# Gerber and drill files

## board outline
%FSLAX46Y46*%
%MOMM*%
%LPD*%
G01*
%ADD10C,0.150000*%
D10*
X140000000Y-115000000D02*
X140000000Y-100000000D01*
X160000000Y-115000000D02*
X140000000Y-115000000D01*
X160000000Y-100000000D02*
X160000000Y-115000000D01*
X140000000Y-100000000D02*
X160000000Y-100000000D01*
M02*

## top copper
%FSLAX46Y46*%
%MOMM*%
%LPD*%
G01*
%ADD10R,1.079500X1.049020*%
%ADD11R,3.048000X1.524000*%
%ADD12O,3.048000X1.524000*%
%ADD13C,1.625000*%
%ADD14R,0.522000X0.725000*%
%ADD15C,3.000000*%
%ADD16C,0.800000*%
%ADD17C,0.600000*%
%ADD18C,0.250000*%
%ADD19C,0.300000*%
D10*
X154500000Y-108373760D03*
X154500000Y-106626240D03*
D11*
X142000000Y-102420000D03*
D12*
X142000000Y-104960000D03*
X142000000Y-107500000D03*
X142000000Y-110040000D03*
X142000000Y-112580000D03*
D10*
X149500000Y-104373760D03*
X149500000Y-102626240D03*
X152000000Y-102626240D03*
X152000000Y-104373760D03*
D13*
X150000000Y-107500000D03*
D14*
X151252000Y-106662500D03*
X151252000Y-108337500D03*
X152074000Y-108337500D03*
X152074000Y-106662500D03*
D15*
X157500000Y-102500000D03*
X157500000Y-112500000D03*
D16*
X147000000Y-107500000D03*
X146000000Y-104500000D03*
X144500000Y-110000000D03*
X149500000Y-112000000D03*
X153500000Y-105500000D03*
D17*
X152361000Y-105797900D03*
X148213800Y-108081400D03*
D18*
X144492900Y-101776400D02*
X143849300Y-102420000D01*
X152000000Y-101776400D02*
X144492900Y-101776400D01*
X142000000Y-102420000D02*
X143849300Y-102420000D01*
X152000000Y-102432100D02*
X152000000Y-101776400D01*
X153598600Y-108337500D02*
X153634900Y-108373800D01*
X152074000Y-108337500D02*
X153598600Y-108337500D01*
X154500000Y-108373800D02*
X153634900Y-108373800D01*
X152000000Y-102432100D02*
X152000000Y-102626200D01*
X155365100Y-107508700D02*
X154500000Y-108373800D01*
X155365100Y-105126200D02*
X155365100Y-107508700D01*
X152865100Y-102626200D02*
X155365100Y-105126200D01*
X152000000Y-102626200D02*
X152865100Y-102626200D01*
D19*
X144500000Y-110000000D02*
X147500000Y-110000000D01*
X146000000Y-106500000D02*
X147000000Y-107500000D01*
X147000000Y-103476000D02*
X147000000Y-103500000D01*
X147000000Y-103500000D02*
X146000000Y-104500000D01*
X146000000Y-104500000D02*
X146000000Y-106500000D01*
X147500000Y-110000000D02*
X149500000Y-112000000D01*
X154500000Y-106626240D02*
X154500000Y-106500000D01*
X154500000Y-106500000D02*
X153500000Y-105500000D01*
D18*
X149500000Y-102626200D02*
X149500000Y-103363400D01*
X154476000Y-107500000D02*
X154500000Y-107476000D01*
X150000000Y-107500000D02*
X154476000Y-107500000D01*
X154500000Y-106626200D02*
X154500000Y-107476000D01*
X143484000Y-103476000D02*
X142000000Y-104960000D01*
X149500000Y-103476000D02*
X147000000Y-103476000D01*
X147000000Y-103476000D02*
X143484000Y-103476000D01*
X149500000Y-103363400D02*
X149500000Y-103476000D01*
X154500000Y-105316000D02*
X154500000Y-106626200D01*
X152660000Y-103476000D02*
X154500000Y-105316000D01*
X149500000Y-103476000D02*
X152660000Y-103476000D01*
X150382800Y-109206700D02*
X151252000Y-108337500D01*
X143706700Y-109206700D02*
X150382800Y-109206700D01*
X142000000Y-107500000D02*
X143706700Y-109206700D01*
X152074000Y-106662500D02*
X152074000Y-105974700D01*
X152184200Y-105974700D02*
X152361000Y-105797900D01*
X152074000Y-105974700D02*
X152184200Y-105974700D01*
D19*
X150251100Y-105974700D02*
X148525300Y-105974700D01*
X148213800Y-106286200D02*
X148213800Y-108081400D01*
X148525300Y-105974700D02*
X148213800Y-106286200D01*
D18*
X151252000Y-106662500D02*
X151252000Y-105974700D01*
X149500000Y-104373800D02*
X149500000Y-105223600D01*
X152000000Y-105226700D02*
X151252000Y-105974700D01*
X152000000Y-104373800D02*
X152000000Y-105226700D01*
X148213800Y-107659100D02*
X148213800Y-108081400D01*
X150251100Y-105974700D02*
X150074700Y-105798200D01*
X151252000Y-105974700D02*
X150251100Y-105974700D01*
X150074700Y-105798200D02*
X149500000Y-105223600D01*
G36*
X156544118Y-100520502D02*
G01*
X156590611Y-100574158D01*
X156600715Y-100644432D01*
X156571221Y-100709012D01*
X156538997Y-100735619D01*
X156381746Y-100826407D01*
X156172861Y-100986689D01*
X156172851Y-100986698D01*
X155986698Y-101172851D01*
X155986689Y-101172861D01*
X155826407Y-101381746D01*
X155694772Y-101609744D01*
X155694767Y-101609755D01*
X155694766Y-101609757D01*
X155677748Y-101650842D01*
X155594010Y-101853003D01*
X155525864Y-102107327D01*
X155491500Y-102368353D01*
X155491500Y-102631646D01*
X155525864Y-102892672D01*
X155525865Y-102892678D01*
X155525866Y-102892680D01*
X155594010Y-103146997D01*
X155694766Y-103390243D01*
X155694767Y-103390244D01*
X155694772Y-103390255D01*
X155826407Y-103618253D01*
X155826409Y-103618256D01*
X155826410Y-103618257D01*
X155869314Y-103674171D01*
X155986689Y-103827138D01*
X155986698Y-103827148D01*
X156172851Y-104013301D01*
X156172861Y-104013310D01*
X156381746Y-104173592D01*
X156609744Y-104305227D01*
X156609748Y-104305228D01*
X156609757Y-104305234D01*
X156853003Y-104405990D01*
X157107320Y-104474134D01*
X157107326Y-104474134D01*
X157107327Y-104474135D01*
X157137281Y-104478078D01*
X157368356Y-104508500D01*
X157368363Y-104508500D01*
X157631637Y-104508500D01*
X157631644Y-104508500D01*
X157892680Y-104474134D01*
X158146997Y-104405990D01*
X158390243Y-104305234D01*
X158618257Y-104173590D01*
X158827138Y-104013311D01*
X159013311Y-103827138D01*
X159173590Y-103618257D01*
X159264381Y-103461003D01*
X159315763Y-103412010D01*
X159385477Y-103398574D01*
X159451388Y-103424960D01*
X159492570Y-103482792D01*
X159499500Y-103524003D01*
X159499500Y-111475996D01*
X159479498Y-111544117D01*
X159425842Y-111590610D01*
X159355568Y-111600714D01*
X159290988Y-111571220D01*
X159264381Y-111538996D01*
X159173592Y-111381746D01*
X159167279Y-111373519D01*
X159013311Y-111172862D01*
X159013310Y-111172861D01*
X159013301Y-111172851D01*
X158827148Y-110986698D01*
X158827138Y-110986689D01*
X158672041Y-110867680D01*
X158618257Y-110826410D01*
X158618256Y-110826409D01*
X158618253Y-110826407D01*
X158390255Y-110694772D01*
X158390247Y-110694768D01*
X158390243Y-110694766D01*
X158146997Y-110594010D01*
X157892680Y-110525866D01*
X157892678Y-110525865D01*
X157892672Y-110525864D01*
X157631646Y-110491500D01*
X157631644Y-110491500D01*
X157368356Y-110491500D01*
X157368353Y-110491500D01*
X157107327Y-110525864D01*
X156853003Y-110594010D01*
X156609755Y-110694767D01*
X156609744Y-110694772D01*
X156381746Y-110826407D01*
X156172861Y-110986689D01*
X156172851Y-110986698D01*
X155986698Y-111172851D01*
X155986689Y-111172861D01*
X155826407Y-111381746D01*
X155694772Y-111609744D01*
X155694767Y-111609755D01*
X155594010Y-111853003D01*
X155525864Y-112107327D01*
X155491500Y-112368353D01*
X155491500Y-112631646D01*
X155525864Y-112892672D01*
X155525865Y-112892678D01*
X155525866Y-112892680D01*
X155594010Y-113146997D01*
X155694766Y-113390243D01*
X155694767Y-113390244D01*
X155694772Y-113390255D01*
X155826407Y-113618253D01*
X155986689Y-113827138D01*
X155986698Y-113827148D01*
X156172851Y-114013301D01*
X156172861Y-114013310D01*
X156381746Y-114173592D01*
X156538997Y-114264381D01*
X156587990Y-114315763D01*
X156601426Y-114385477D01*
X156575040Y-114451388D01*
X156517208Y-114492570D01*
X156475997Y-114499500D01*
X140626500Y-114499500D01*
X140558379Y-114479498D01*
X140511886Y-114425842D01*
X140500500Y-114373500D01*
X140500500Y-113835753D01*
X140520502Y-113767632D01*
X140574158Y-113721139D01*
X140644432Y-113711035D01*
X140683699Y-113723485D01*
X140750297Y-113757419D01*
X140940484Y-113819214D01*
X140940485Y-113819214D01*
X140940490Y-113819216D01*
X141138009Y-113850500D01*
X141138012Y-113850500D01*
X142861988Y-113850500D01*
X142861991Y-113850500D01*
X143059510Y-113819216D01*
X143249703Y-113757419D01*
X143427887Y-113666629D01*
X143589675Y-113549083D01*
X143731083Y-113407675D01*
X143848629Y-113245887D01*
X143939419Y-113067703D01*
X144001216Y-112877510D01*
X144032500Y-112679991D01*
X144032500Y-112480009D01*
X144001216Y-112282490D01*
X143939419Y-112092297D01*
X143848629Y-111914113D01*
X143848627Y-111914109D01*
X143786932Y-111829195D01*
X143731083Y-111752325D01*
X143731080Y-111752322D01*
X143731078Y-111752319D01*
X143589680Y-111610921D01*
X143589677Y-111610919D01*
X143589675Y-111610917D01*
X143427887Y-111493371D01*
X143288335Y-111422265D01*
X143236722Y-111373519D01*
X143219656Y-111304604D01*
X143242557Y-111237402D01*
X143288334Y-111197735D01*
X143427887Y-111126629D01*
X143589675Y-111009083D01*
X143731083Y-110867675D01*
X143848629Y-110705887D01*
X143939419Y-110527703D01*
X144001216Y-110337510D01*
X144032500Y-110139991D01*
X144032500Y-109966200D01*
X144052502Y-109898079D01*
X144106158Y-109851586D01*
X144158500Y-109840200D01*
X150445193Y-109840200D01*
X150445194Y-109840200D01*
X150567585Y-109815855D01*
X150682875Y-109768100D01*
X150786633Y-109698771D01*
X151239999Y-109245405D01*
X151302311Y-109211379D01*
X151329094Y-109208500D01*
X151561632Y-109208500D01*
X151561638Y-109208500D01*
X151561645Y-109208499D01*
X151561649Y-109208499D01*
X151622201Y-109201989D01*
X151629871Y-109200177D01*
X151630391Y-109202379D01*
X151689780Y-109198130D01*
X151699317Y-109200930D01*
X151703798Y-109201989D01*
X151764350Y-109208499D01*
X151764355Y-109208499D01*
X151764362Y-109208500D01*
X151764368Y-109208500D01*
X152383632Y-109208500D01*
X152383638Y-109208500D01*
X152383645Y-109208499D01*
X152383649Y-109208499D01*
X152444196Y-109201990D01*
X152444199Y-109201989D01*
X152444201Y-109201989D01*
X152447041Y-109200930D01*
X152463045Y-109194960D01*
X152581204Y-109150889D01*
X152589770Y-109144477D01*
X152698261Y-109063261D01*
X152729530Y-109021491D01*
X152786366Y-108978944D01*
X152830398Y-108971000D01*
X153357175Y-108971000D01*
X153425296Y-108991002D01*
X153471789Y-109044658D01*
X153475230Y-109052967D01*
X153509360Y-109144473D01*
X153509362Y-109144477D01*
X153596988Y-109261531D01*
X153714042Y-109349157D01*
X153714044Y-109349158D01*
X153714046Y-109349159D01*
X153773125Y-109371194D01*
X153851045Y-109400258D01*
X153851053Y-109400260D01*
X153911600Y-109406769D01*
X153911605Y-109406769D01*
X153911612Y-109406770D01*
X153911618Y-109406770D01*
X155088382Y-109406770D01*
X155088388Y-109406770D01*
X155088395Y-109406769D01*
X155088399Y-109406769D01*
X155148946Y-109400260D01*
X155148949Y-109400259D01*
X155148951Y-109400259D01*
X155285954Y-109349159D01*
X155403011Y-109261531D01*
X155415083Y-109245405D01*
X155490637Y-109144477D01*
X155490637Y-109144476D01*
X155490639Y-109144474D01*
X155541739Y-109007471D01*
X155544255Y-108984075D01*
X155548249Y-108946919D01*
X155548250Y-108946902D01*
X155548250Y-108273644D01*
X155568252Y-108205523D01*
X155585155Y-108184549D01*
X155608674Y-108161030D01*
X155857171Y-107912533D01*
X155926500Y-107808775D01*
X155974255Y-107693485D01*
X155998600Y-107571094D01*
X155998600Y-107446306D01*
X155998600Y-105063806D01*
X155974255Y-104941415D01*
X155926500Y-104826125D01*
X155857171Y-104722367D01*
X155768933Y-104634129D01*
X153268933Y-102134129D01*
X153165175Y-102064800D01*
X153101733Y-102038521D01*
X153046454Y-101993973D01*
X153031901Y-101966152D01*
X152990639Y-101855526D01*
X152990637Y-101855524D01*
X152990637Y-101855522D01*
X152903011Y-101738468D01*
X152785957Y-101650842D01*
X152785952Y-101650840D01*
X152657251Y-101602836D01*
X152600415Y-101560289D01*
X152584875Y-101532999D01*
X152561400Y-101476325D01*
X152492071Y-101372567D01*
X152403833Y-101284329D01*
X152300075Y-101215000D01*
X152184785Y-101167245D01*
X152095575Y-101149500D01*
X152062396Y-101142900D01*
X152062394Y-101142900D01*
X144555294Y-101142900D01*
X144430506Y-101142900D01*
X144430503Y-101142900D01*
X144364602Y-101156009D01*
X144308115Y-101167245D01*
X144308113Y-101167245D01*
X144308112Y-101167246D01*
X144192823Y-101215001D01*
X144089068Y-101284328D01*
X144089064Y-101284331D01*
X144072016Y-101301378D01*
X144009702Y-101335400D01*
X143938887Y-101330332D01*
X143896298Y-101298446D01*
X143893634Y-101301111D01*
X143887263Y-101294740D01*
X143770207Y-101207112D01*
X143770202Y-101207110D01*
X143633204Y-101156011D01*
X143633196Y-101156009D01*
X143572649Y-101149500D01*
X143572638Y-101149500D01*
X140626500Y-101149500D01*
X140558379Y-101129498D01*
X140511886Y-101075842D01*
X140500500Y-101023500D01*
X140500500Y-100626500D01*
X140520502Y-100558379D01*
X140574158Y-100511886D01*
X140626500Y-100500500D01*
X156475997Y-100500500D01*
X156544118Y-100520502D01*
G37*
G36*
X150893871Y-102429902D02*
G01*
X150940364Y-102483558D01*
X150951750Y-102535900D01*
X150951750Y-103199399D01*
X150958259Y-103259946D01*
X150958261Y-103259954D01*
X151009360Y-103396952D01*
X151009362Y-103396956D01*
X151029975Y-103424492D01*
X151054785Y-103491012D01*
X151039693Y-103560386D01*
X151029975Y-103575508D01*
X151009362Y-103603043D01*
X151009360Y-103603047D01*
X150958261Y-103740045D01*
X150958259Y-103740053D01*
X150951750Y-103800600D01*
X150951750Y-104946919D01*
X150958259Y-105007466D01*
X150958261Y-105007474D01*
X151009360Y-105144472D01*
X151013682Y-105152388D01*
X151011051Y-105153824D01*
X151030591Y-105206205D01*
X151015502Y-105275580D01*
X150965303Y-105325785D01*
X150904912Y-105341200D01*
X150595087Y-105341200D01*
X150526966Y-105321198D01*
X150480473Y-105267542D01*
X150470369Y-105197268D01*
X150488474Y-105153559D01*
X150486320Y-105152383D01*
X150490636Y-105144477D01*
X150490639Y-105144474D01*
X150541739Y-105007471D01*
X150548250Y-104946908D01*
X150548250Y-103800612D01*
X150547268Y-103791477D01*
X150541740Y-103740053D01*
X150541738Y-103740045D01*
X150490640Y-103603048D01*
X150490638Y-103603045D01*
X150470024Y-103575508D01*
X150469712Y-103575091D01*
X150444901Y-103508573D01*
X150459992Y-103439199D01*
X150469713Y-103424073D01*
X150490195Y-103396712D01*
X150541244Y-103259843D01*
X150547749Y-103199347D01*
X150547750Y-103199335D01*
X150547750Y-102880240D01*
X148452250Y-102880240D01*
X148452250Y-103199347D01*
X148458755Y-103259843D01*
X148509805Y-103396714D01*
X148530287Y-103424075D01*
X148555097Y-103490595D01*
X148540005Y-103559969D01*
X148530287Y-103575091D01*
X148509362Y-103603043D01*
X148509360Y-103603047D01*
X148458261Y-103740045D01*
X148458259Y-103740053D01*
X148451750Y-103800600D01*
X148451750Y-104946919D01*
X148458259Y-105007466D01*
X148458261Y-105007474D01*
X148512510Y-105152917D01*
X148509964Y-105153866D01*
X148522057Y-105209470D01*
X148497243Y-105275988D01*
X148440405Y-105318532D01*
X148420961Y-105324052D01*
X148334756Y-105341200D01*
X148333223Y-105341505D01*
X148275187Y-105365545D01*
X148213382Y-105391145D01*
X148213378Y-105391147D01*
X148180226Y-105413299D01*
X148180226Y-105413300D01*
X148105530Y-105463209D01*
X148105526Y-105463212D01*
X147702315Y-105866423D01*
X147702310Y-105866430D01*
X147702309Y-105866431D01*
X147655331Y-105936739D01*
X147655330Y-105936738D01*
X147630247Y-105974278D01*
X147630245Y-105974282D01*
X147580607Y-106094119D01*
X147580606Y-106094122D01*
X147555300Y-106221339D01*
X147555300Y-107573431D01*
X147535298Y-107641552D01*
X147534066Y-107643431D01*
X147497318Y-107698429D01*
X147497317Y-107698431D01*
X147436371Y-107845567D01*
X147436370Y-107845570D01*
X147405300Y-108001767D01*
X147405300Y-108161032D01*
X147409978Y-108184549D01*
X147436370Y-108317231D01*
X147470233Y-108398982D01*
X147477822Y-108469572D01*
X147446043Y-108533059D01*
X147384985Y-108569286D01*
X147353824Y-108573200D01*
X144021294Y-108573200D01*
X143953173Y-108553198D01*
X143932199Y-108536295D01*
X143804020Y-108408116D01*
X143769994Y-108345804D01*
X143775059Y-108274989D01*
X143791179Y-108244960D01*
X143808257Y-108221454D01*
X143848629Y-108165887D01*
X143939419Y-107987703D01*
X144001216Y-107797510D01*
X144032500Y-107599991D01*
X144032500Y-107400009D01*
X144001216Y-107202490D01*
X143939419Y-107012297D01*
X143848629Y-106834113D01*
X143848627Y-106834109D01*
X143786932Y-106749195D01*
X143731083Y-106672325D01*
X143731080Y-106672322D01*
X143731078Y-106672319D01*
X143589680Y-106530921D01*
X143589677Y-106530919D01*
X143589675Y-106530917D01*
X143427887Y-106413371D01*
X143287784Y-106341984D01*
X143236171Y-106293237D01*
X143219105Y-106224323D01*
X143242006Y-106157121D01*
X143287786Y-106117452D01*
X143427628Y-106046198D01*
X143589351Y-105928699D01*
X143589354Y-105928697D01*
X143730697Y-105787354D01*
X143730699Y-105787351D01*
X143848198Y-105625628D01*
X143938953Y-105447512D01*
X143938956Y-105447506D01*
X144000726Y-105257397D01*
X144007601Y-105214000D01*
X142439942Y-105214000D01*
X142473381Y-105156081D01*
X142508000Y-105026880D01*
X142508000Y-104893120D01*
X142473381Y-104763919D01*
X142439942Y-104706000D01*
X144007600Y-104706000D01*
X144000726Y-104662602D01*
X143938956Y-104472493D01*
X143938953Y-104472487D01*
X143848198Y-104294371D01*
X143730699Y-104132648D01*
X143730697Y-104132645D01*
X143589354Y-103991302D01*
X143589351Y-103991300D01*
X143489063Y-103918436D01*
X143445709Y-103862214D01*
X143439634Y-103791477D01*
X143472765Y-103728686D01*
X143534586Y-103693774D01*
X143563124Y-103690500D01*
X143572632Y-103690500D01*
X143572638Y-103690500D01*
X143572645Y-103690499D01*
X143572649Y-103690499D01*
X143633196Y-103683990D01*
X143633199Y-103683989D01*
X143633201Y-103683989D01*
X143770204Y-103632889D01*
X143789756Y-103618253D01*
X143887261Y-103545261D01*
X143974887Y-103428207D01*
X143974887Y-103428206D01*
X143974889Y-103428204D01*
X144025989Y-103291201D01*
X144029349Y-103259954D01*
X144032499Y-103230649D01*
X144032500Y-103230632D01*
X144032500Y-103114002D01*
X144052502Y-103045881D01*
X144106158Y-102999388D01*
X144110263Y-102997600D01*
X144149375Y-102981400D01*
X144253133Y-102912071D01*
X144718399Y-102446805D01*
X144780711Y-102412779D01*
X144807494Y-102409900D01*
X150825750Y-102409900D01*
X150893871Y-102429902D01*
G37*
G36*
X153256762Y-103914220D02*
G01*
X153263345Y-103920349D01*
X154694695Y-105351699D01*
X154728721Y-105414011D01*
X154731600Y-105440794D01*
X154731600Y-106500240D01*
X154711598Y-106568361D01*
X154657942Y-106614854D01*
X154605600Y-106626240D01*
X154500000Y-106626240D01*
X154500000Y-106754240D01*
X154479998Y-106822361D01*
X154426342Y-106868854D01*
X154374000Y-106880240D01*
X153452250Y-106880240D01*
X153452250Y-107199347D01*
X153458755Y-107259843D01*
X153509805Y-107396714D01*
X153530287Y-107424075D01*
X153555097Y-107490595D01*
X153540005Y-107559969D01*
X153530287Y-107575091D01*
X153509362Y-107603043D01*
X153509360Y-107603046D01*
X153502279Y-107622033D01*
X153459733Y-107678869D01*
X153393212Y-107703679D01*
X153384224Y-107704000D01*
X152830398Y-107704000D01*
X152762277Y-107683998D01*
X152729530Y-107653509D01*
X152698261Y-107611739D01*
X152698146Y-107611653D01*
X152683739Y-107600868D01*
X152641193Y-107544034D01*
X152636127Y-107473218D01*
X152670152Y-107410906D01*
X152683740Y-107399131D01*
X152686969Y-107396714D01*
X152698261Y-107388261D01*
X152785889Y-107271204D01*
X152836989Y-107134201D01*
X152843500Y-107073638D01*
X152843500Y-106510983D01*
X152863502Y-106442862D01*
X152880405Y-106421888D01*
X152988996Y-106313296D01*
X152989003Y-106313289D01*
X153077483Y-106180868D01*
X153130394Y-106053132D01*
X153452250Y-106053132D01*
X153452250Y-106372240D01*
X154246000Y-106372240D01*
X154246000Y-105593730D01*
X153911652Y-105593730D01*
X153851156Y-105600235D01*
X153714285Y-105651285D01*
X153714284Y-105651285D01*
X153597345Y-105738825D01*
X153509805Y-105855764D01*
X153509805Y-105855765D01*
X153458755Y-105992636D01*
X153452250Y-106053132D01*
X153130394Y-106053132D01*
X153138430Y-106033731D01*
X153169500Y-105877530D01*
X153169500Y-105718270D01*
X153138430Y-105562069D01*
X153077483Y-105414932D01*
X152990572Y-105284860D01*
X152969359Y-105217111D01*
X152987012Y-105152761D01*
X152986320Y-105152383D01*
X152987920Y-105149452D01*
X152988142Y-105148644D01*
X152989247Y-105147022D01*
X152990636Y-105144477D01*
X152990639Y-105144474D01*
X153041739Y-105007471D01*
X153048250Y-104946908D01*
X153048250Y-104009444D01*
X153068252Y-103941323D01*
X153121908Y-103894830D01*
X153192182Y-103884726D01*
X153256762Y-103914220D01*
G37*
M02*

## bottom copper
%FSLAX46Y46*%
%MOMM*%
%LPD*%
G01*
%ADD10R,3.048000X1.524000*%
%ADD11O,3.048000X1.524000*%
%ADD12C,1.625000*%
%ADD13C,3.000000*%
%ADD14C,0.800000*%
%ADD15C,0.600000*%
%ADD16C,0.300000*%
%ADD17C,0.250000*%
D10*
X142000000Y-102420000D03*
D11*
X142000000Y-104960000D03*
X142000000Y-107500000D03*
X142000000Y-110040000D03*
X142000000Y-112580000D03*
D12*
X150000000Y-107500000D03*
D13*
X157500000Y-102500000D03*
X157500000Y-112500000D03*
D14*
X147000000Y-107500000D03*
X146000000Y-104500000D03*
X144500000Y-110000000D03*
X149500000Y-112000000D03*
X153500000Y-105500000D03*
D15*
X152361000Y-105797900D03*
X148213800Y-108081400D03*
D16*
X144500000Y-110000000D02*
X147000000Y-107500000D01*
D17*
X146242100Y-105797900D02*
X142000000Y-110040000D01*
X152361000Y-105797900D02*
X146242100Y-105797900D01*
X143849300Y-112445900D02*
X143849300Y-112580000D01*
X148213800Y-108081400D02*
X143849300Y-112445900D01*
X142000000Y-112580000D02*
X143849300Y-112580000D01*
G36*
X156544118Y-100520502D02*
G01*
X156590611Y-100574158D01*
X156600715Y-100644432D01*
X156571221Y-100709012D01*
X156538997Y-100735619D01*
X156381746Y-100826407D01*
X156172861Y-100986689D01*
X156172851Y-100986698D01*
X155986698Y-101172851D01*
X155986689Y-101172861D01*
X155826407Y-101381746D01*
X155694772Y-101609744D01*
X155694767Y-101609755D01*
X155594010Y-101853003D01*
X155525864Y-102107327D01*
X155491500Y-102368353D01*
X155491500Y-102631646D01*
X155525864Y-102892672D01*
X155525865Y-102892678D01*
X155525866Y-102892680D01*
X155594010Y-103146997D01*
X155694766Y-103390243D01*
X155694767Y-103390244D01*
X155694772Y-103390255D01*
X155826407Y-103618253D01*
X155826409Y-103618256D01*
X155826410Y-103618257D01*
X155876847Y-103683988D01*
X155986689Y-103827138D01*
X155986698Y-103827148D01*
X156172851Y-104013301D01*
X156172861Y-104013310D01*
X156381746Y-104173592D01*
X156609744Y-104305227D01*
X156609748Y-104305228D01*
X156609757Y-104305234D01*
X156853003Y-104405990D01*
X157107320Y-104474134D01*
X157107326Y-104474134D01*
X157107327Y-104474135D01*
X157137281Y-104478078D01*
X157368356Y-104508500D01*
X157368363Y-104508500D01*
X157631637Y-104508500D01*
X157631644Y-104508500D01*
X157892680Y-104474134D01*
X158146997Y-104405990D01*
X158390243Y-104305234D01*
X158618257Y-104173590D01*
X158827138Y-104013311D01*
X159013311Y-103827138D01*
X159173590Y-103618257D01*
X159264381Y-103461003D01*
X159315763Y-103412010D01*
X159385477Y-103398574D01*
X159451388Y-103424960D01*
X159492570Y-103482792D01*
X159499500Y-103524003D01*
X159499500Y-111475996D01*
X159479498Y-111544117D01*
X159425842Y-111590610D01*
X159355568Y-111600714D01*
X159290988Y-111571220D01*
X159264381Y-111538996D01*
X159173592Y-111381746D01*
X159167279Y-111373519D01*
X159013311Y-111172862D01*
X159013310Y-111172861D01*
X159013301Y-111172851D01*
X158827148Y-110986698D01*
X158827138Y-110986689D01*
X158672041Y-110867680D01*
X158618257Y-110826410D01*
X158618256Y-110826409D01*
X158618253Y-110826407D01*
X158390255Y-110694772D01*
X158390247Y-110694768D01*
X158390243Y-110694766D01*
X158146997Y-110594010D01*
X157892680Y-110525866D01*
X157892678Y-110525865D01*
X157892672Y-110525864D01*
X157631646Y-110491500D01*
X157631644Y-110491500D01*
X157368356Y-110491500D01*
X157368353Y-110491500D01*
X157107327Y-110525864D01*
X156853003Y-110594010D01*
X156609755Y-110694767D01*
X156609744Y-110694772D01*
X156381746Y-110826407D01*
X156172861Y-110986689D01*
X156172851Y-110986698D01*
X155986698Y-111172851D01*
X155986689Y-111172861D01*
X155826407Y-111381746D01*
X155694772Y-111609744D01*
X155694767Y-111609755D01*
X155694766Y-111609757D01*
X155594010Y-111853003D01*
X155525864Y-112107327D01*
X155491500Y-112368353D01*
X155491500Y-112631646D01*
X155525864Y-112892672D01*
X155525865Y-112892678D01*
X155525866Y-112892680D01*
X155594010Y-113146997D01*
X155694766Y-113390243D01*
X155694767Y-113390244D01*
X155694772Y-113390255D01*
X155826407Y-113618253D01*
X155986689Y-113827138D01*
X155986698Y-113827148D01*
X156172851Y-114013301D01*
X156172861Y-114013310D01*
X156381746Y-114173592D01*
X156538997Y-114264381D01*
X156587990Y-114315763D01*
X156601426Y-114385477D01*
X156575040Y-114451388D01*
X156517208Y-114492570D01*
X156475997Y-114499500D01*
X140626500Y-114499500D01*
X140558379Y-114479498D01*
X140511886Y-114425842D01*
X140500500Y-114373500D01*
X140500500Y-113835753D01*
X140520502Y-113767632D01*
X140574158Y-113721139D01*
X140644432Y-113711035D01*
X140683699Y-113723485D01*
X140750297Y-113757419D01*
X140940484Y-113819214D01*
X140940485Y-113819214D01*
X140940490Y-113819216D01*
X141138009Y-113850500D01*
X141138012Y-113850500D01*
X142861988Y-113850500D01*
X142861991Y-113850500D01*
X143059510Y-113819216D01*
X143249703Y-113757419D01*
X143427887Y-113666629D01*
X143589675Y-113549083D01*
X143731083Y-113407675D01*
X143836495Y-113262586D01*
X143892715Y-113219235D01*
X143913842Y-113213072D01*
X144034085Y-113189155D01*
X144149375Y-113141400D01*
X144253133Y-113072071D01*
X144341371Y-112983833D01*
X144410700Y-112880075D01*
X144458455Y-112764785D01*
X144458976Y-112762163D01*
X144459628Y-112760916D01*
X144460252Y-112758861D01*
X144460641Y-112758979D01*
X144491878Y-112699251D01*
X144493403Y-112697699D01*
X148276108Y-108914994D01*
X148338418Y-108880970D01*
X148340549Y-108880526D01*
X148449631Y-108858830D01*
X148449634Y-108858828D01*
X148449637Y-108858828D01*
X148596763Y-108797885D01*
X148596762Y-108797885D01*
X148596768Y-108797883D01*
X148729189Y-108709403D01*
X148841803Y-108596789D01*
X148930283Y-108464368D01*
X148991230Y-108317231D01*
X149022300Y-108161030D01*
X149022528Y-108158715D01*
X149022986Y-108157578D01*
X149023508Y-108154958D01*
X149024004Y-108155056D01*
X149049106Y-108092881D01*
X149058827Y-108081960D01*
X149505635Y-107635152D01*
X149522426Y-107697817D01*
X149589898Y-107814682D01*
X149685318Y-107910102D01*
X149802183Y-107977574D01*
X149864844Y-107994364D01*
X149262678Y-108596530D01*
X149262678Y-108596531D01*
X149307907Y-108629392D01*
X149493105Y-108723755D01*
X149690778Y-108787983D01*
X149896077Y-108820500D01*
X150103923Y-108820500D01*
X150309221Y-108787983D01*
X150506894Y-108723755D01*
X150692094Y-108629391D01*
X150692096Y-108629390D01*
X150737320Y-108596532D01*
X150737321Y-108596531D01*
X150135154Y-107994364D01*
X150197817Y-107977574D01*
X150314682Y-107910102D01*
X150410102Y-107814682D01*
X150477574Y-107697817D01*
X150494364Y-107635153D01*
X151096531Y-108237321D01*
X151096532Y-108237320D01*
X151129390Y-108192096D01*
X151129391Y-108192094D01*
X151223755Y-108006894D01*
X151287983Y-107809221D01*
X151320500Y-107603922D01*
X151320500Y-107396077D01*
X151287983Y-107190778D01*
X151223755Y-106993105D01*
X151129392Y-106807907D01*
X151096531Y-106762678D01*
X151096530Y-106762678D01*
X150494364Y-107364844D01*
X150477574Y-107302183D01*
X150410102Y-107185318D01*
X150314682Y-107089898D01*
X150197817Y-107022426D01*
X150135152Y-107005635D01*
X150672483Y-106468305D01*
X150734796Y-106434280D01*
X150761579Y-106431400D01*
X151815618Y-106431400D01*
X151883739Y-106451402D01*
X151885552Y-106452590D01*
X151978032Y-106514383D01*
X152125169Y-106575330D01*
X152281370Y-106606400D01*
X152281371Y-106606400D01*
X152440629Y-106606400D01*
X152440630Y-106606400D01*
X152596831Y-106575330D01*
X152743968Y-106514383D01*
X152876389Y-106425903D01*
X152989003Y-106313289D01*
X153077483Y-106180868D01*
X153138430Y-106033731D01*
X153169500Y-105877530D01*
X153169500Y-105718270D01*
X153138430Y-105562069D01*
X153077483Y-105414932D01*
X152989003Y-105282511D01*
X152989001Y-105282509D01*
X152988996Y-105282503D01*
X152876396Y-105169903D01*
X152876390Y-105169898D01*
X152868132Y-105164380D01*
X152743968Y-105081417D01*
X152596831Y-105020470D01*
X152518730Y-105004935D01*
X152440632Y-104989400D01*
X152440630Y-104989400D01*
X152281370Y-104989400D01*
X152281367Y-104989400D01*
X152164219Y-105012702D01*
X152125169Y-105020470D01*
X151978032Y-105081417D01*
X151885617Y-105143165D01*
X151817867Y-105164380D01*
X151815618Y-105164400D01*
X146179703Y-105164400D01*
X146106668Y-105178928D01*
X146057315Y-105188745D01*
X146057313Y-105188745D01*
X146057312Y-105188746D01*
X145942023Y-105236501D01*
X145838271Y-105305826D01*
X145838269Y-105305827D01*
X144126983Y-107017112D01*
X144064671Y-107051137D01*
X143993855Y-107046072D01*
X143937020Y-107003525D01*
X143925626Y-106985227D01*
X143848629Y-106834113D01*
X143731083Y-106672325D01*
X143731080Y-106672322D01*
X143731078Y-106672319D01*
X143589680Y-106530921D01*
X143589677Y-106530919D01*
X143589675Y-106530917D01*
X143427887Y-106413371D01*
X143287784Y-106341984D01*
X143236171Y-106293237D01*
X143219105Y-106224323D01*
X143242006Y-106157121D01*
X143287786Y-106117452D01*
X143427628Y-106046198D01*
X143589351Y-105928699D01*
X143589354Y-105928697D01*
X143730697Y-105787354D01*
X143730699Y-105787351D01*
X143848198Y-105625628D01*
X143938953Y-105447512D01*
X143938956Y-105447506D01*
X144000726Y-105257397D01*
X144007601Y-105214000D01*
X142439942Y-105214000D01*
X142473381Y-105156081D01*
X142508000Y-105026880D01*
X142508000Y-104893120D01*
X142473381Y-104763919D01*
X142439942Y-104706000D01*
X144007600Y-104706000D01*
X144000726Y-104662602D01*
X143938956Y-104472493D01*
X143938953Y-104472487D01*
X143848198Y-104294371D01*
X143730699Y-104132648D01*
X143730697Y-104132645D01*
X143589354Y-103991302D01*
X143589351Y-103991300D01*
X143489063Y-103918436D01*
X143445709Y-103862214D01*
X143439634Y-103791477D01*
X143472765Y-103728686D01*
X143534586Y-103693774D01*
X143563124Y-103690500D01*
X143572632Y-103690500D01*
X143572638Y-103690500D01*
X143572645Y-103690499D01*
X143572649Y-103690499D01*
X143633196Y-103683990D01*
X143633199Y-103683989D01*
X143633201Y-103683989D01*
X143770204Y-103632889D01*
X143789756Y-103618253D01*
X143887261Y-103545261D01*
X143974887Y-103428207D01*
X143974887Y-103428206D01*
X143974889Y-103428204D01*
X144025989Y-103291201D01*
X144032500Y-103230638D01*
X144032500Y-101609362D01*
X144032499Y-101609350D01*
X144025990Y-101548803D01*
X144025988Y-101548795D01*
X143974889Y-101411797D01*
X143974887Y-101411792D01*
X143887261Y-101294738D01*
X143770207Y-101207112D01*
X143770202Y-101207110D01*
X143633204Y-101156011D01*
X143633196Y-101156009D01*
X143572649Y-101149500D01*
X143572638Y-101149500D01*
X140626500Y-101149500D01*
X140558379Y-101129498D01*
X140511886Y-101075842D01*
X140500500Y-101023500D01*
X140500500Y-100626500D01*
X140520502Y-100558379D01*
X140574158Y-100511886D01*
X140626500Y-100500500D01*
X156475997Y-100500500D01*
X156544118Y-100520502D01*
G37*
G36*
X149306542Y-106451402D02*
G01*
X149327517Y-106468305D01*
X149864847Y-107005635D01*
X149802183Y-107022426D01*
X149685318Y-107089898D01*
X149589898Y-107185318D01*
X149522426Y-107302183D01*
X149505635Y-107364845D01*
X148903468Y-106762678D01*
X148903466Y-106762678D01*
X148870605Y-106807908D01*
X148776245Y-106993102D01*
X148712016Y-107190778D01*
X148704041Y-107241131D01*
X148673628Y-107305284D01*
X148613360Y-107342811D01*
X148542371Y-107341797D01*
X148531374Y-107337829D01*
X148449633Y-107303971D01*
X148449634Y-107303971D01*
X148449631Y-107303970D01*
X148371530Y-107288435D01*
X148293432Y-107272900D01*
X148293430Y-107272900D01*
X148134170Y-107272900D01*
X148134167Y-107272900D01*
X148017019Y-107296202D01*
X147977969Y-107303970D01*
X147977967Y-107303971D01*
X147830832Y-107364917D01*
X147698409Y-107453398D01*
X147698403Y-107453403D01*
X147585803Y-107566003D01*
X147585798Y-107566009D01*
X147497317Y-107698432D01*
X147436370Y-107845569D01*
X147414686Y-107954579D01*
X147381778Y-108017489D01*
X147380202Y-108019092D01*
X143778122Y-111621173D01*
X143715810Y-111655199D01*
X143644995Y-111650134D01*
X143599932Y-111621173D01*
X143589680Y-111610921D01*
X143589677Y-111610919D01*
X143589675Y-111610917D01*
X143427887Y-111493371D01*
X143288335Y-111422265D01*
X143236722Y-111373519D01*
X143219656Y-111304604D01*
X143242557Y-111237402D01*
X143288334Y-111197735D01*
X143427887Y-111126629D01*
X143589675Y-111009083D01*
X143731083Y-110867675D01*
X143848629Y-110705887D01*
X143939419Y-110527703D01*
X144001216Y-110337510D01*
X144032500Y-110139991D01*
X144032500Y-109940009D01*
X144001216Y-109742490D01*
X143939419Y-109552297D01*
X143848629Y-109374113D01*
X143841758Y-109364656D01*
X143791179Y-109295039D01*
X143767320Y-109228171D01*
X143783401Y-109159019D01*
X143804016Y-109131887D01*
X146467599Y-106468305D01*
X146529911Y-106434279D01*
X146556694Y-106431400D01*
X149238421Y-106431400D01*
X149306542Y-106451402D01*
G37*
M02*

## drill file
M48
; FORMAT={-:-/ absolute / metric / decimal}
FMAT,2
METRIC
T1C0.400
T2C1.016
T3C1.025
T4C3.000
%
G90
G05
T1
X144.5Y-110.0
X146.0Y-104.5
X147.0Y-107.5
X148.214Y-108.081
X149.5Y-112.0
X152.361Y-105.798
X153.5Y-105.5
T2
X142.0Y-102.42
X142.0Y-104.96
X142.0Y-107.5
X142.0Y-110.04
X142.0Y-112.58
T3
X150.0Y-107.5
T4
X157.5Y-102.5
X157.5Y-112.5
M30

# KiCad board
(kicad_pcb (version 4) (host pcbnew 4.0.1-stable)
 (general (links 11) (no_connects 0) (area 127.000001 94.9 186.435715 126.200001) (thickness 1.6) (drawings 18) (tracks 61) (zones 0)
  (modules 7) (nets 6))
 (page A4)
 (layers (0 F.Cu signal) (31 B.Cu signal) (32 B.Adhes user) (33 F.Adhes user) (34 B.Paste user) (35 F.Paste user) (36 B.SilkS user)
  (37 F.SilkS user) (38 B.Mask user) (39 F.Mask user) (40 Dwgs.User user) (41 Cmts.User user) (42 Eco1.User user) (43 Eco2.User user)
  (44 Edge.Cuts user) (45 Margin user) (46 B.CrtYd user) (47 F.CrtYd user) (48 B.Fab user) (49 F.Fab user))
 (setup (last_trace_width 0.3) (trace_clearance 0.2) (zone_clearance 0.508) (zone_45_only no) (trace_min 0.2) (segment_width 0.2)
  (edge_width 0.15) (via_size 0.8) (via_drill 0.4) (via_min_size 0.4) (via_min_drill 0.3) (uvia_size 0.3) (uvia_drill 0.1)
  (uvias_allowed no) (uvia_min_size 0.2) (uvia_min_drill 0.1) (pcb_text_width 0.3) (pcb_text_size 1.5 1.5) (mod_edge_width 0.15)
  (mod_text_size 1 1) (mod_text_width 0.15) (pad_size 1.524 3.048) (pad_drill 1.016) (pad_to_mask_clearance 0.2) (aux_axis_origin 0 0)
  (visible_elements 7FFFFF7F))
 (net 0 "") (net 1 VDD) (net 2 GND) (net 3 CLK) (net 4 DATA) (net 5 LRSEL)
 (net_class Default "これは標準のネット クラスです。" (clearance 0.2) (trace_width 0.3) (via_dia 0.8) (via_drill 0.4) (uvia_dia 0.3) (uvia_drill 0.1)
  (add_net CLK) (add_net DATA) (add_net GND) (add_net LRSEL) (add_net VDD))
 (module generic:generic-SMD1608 (layer F.Cu) (at 154.5 107.5 90)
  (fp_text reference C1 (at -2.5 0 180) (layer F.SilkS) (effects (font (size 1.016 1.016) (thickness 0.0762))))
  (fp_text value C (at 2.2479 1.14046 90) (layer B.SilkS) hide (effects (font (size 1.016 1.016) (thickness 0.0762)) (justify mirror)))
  (pad 1 smd rect (at -0.87376 0 90) (size 1.04902 1.0795) (layers F.Cu F.Paste F.Mask) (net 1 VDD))
  (pad 2 smd rect (at 0.87376 0 90) (size 1.04902 1.0795) (layers F.Cu F.Paste F.Mask) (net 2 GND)))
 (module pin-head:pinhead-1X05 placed (layer F.Cu) (at 142 107.5 270)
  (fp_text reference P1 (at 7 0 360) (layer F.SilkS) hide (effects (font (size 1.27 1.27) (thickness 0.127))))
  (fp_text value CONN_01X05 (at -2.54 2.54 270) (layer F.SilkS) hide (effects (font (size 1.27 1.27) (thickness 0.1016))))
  (pad 1 thru_hole rect (at -5.08 0 90) (size 1.524 3.048) (drill 1.016) (layers *.Cu *.Paste *.Mask F.SilkS) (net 1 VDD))
  (pad 2 thru_hole oval (at -2.54 0 90) (size 1.524 3.048) (drill 1.016) (layers *.Cu *.Paste *.Mask F.SilkS) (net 2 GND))
  (pad 3 thru_hole oval (at 0 0 90) (size 1.524 3.048) (drill 1.016) (layers *.Cu *.Paste *.Mask F.SilkS) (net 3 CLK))
  (pad 4 thru_hole oval (at 2.54 0 90) (size 1.524 3.048) (drill 1.016) (layers *.Cu *.Paste *.Mask F.SilkS) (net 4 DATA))
  (pad 5 thru_hole oval (at 5.08 0 90) (size 1.524 3.048) (drill 1.016) (layers *.Cu *.Paste *.Mask F.SilkS) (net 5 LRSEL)))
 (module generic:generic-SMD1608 (layer F.Cu) (at 149.5 103.5 90)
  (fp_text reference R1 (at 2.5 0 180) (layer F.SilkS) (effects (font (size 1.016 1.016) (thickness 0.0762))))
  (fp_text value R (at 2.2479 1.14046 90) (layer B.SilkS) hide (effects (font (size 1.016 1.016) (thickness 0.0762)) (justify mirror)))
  (pad 1 smd rect (at -0.87376 0 90) (size 1.04902 1.0795) (layers F.Cu F.Paste F.Mask) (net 5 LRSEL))
  (pad 2 smd rect (at 0.87376 0 90) (size 1.04902 1.0795) (layers F.Cu F.Paste F.Mask) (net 2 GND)))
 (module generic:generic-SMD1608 (layer F.Cu) (at 152 103.5 270)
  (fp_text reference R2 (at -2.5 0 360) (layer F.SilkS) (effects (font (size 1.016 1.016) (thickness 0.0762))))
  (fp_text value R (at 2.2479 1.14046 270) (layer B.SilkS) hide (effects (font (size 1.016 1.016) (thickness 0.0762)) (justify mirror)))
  (pad 1 smd rect (at -0.87376 0 270) (size 1.04902 1.0795) (layers F.Cu F.Paste F.Mask) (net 1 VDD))
  (pad 2 smd rect (at 0.87376 0 270) (size 1.04902 1.0795) (layers F.Cu F.Paste F.Mask) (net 5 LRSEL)))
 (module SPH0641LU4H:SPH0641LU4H (layer F.Cu) (at 150 107.5 270)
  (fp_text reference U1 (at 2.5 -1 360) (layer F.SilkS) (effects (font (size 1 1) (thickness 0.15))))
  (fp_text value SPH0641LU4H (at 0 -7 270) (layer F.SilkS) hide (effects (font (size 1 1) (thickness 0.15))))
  (pad 3 thru_hole circle (at 0 0 270) (size 1.625 1.625) (drill 1.025) (layers *.Cu *.Mask F.SilkS) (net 2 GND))
  (pad 2 smd rect (at -0.8375 -1.252 270) (size 0.725 0.522) (layers F.Cu F.Paste F.Mask) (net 5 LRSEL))
  (pad 4 smd rect (at 0.8375 -1.252 270) (size 0.725 0.522) (layers F.Cu F.Paste F.Mask) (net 3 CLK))
  (pad 5 smd rect (at 0.8375 -2.074 270) (size 0.725 0.522) (layers F.Cu F.Paste F.Mask) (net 1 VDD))
  (pad 1 smd rect (at -0.8375 -2.074 270) (size 0.725 0.522) (layers F.Cu F.Paste F.Mask) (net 4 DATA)))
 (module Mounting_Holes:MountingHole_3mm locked (layer F.Cu) (at 157.5 102.5)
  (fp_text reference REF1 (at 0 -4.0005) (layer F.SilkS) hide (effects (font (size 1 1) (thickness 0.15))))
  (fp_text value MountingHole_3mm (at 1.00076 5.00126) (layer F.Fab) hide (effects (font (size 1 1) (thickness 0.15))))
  (pad 1 thru_hole circle (at 0 0) (size 3 3) (drill 3) (layers)))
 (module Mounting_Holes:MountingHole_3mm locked (layer F.Cu) (at 157.5 112.5)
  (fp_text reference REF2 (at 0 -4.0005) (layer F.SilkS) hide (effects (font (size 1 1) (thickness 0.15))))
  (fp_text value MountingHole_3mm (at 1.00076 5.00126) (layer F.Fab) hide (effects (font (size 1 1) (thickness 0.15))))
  (pad 1 thru_hole circle (at 0 0) (size 3 3) (drill 3) (layers)))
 (gr_line (start 140 115) (end 140 100) (angle 90) (layer Edge.Cuts) (width 0.15))
 (gr_line (start 160 115) (end 140 115) (angle 90) (layer Edge.Cuts) (width 0.15))
 (gr_line (start 160 100) (end 160 115) (angle 90) (layer Edge.Cuts) (width 0.15))
 (gr_line (start 140 100) (end 160 100) (angle 90) (layer Edge.Cuts) (width 0.15))
 (segment (start 144.4929 101.7764) (end 143.8493 102.42) (width 0.25) (layer F.Cu) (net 1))
 (segment (start 152 101.7764) (end 144.4929 101.7764) (width 0.25) (layer F.Cu) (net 1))
 (segment (start 142 102.42) (end 143.8493 102.42) (width 0.25) (layer F.Cu) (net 1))
 (segment (start 152 102.4321) (end 152 101.7764) (width 0.25) (layer F.Cu) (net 1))
 (segment (start 153.5986 108.3375) (end 153.6349 108.3738) (width 0.25) (layer F.Cu) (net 1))
 (segment (start 152.074 108.3375) (end 153.5986 108.3375) (width 0.25) (layer F.Cu) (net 1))
 (segment (start 154.5 108.3738) (end 153.6349 108.3738) (width 0.25) (layer F.Cu) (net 1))
 (segment (start 152 102.4321) (end 152 102.6262) (width 0.25) (layer F.Cu) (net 1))
 (segment (start 155.3651 107.5087) (end 154.5 108.3738) (width 0.25) (layer F.Cu) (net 1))
 (segment (start 155.3651 105.1262) (end 155.3651 107.5087) (width 0.25) (layer F.Cu) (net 1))
 (segment (start 152.8651 102.6262) (end 155.3651 105.1262) (width 0.25) (layer F.Cu) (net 1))
 (segment (start 152 102.6262) (end 152.8651 102.6262) (width 0.25) (layer F.Cu) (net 1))
 (segment (start 144.5 110) (end 147.5 110) (width 0.3) (layer F.Cu) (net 2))
 (segment (start 144.5 110) (end 147 107.5) (width 0.3) (layer B.Cu) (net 2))
 (segment (start 146 106.5) (end 147 107.5) (width 0.3) (layer F.Cu) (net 2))
 (via (at 147 107.5) (size 0.8) (drill 0.4) (layers F.Cu B.Cu) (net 2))
 (segment (start 147 103.476) (end 147 103.5) (width 0.3) (layer F.Cu) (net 2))
 (via (at 146 104.5) (size 0.8) (drill 0.4) (layers F.Cu B.Cu) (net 2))
 (segment (start 147 103.5) (end 146 104.5) (width 0.3) (layer F.Cu) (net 2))
 (segment (start 146 104.5) (end 146 106.5) (width 0.3) (layer F.Cu) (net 2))
 (via (at 144.5 110) (size 0.8) (drill 0.4) (layers F.Cu B.Cu) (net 2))
 (via (at 149.5 112) (size 0.8) (drill 0.4) (layers F.Cu B.Cu) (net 2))
 (segment (start 147.5 110) (end 149.5 112) (width 0.3) (layer F.Cu) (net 2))
 (segment (start 154.5 106.62624) (end 154.5 106.5) (width 0.3) (layer F.Cu) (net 2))
 (segment (start 154.5 106.5) (end 153.5 105.5) (width 0.3) (layer F.Cu) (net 2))
 (via (at 153.5 105.5) (size 0.8) (drill 0.4) (layers F.Cu B.Cu) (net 2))
 (segment (start 149.5 102.6262) (end 149.5 103.3634) (width 0.25) (layer F.Cu) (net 2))
 (segment (start 154.476 107.5) (end 154.5 107.476) (width 0.25) (layer F.Cu) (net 2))
 (segment (start 150 107.5) (end 154.476 107.5) (width 0.25) (layer F.Cu) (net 2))
 (segment (start 154.5 106.6262) (end 154.5 107.476) (width 0.25) (layer F.Cu) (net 2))
 (segment (start 143.484 103.476) (end 142 104.96) (width 0.25) (layer F.Cu) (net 2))
 (segment (start 149.5 103.476) (end 147 103.476) (width 0.25) (layer F.Cu) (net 2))
 (segment (start 147 103.476) (end 143.484 103.476) (width 0.25) (layer F.Cu) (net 2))
 (segment (start 149.5 103.3634) (end 149.5 103.476) (width 0.25) (layer F.Cu) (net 2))
 (segment (start 154.5 105.316) (end 154.5 106.6262) (width 0.25) (layer F.Cu) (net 2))
 (segment (start 152.66 103.476) (end 154.5 105.316) (width 0.25) (layer F.Cu) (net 2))
 (segment (start 149.5 103.476) (end 152.66 103.476) (width 0.25) (layer F.Cu) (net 2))
 (segment (start 150.3828 109.2067) (end 151.252 108.3375) (width 0.25) (layer F.Cu) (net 3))
 (segment (start 143.7067 109.2067) (end 150.3828 109.2067) (width 0.25) (layer F.Cu) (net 3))
 (segment (start 142 107.5) (end 143.7067 109.2067) (width 0.25) (layer F.Cu) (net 3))
 (via (at 152.361 105.7979) (size 0.6) (layers F.Cu B.Cu) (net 4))
 (segment (start 152.074 106.6625) (end 152.074 105.9747) (width 0.25) (layer F.Cu) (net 4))
 (segment (start 146.2421 105.7979) (end 142 110.04) (width 0.25) (layer B.Cu) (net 4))
 (segment (start 152.361 105.7979) (end 146.2421 105.7979) (width 0.25) (layer B.Cu) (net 4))
 (segment (start 152.1842 105.9747) (end 152.361 105.7979) (width 0.25) (layer F.Cu) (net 4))
 (segment (start 152.074 105.9747) (end 152.1842 105.9747) (width 0.25) (layer F.Cu) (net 4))
 (segment (start 150.2511 105.9747) (end 148.5253 105.9747) (width 0.3) (layer F.Cu) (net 5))
 (segment (start 148.2138 106.2862) (end 148.2138 108.0814) (width 0.3) (layer F.Cu) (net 5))
 (segment (start 148.5253 105.9747) (end 148.2138 106.2862) (width 0.3) (layer F.Cu) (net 5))
 (via (at 148.2138 108.0814) (size 0.6) (layers F.Cu B.Cu) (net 5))
 (segment (start 143.8493 112.4459) (end 143.8493 112.58) (width 0.25) (layer B.Cu) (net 5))
 (segment (start 148.2138 108.0814) (end 143.8493 112.4459) (width 0.25) (layer B.Cu) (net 5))
 (segment (start 142 112.58) (end 143.8493 112.58) (width 0.25) (layer B.Cu) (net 5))
 (segment (start 151.252 106.6625) (end 151.252 105.9747) (width 0.25) (layer F.Cu) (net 5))
 (segment (start 149.5 104.3738) (end 149.5 105.2236) (width 0.25) (layer F.Cu) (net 5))
 (segment (start 152 105.2267) (end 151.252 105.9747) (width 0.25) (layer F.Cu) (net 5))
 (segment (start 152 104.3738) (end 152 105.2267) (width 0.25) (layer F.Cu) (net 5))
 (segment (start 148.2138 107.6591) (end 148.2138 108.0814) (width 0.25) (layer F.Cu) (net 5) (status 2))
 (segment (start 150.2511 105.9747) (end 150.0747 105.7982) (width 0.25) (layer F.Cu) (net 5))
 (segment (start 151.252 105.9747) (end 150.2511 105.9747) (width 0.25) (layer F.Cu) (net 5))
 (segment (start 150.0747 105.7982) (end 149.5 105.2236) (width 0.25) (layer F.Cu) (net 5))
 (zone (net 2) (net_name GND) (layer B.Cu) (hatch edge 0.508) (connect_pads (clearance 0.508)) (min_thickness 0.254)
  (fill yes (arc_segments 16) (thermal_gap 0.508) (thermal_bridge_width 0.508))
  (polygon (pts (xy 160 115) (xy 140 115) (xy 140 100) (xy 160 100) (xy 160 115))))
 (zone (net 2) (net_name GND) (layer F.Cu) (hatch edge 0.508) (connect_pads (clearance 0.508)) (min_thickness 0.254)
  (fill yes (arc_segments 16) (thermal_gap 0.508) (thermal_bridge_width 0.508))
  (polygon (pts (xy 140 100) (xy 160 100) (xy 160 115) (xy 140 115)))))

